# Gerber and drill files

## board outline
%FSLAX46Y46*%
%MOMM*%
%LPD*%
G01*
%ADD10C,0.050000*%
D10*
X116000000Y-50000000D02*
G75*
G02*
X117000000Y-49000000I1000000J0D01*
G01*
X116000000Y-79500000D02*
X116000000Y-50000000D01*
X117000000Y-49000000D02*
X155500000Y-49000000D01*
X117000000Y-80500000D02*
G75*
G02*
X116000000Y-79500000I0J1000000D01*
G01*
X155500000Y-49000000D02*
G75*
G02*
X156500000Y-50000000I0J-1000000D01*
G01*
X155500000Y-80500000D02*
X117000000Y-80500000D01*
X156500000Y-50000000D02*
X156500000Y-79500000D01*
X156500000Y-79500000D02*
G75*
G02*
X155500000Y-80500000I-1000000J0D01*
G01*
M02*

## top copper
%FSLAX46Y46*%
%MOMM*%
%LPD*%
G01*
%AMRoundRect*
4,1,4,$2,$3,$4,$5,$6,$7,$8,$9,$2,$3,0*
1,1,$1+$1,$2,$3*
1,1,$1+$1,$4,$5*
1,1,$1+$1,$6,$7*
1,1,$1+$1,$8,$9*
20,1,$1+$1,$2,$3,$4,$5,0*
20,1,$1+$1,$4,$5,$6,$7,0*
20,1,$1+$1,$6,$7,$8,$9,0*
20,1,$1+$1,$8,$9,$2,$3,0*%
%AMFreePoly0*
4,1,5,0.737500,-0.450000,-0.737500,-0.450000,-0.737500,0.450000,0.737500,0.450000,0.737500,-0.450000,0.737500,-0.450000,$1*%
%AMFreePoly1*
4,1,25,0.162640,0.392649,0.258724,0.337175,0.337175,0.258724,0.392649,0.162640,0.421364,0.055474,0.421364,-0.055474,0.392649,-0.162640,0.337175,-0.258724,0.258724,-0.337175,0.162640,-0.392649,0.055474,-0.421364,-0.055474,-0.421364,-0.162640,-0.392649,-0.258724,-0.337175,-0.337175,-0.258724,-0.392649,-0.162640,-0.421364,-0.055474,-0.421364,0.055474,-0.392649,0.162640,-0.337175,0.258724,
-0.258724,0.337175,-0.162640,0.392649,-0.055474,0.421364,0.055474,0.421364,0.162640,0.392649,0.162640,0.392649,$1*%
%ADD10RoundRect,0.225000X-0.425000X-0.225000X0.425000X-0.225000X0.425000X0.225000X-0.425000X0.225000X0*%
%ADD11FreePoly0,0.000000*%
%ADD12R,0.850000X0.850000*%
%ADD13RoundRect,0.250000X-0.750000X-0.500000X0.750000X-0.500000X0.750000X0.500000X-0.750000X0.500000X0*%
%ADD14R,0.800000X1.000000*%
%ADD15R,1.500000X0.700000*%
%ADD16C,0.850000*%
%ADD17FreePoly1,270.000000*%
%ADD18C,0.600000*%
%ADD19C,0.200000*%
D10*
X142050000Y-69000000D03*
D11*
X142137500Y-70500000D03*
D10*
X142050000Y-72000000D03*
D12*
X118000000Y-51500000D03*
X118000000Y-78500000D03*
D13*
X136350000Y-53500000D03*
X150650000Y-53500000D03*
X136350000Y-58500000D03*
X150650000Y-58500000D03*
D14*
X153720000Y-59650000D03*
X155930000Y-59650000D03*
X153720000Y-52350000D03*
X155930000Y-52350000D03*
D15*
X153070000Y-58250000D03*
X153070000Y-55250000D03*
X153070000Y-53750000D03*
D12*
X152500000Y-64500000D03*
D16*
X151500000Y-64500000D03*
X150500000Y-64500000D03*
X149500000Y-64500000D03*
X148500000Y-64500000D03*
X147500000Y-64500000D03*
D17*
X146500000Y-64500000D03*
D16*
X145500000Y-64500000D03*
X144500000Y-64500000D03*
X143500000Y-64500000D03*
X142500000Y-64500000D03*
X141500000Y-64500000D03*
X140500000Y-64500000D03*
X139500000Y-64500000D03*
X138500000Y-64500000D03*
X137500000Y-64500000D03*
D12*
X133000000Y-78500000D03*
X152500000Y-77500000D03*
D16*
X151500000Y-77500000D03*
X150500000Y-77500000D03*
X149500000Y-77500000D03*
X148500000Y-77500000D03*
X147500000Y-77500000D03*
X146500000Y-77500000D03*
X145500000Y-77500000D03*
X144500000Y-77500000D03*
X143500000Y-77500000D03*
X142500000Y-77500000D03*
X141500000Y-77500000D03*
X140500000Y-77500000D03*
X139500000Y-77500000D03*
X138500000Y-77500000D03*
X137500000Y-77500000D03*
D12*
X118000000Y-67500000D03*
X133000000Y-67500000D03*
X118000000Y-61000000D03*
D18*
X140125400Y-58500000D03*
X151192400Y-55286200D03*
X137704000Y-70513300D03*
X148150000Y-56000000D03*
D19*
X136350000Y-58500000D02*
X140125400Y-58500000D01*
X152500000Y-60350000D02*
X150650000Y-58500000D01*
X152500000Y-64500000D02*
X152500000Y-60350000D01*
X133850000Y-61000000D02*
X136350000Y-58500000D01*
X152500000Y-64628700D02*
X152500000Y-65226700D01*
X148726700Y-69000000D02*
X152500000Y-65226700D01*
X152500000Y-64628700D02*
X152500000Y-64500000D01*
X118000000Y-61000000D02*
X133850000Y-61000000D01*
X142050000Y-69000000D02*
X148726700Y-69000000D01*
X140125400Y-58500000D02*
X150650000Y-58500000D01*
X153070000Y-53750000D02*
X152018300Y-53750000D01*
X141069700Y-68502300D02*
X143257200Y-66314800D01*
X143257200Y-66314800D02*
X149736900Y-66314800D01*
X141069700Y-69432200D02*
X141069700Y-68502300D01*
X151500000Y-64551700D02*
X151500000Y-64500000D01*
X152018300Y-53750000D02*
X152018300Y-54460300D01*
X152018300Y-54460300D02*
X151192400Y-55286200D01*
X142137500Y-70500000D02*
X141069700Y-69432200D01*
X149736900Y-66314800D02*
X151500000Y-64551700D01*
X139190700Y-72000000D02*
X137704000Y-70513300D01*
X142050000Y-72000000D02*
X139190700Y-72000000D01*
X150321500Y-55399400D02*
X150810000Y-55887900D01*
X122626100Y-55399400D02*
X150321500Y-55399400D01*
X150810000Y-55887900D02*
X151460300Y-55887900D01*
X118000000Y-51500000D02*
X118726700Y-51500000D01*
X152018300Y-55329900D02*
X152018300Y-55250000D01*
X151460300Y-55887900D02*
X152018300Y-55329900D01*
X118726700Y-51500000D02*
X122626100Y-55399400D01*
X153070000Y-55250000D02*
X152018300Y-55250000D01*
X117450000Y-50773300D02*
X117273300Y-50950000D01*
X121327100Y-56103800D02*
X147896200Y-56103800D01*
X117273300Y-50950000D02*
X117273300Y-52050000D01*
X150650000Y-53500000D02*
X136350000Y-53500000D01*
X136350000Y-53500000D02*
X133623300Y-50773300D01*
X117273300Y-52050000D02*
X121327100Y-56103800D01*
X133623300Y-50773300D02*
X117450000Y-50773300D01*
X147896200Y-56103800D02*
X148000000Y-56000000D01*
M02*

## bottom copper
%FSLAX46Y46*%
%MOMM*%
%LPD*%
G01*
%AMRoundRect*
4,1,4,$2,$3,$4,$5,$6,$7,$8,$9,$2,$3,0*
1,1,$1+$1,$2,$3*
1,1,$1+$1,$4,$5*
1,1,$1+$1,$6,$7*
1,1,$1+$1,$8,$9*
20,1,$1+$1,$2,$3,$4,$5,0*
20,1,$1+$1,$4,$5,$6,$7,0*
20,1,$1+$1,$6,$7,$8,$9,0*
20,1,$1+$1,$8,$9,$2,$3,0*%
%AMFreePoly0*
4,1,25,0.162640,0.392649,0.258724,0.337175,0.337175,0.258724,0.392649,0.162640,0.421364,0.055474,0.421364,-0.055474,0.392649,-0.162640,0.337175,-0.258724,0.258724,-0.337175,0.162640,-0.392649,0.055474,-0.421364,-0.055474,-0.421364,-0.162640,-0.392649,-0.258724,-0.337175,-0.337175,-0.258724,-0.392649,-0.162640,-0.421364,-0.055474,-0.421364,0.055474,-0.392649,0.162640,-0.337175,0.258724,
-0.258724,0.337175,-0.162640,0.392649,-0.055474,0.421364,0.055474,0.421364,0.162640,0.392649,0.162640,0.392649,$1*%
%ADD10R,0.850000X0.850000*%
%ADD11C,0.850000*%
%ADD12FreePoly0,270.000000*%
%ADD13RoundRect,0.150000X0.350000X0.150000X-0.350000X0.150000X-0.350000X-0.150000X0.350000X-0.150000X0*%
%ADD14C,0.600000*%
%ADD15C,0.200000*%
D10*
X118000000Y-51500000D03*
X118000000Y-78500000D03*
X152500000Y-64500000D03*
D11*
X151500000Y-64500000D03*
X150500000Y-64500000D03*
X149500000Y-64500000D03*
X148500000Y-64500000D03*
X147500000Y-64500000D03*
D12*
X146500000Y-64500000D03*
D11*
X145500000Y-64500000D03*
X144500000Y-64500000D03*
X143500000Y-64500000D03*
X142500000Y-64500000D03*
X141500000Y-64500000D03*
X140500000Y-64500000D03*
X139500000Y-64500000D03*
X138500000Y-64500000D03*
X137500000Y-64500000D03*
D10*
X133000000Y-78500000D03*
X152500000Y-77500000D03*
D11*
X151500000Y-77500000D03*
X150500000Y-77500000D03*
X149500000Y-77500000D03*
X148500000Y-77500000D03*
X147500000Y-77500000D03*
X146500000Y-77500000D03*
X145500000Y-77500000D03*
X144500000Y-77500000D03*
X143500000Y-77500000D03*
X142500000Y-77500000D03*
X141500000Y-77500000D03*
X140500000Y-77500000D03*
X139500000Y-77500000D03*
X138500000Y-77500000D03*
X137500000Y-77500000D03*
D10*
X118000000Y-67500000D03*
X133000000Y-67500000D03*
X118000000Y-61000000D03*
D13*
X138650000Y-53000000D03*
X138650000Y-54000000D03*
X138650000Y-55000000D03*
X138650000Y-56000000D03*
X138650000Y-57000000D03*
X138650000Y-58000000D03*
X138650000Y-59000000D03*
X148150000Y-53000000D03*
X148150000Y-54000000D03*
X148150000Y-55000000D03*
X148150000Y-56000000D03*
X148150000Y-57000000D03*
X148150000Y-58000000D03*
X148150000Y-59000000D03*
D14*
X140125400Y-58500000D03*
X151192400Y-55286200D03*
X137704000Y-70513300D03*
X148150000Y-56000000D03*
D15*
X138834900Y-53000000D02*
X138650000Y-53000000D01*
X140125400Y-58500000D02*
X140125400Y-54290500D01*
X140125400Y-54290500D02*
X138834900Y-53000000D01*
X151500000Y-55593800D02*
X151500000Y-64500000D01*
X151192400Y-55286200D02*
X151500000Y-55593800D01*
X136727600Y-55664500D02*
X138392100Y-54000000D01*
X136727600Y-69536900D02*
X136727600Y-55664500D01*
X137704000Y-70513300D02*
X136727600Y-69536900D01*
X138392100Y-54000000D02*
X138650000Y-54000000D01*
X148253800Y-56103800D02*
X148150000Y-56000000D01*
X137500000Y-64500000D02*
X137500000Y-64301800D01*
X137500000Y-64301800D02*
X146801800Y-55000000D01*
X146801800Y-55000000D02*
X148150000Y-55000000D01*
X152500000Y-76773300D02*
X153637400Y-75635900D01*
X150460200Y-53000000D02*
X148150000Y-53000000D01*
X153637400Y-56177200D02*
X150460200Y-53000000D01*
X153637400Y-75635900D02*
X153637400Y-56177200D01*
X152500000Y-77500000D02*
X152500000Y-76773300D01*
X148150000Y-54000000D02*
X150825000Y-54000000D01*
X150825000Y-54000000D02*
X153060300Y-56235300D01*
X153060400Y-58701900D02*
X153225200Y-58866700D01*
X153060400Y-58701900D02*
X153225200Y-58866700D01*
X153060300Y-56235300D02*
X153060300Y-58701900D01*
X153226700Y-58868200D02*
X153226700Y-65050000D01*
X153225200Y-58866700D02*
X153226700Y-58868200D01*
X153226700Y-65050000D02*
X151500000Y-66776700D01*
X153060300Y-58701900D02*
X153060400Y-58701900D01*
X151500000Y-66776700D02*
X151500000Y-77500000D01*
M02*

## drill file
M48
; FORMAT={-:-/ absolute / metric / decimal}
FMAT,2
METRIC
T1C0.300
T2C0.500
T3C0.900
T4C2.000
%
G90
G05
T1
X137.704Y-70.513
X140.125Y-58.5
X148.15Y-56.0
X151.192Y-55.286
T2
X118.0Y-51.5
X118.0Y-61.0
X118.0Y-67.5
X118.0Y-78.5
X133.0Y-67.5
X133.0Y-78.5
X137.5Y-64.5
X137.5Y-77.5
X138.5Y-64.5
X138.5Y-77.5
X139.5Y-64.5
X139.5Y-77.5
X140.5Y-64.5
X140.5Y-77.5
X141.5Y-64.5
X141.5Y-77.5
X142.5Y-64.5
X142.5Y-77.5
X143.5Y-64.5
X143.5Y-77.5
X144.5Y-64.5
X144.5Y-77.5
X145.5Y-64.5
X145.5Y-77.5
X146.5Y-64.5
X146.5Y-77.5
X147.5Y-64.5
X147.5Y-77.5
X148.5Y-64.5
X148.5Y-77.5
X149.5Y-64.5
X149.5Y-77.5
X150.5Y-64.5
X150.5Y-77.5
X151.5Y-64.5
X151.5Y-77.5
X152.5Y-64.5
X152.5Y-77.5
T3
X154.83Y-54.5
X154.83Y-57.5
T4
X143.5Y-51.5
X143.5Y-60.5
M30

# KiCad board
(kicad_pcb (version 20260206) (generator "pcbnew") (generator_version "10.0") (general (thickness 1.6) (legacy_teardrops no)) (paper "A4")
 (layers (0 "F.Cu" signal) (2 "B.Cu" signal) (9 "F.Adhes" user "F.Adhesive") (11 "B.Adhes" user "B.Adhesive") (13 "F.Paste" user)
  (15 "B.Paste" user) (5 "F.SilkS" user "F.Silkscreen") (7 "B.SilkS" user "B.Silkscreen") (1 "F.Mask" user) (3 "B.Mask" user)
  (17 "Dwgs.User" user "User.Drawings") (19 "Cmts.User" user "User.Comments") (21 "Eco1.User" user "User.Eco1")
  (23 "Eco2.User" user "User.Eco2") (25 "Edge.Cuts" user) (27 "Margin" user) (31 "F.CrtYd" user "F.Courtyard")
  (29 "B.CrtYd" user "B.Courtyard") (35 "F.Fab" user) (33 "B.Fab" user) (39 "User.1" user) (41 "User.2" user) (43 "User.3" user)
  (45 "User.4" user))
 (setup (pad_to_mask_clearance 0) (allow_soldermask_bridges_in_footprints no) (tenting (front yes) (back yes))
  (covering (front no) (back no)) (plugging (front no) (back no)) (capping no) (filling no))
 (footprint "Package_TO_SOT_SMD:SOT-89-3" (layer "F.Cu") (at 144 70.5)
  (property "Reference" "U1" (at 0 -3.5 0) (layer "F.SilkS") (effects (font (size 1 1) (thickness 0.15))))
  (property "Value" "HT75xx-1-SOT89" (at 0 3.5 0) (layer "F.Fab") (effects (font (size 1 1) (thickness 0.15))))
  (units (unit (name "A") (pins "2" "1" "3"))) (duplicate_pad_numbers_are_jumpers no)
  (pad "1" smd roundrect (at -1.95 -1.5) (size 1.3 0.9) (layers "F.Cu" "F.Mask" "F.Paste") (roundrect_rratio 0.25) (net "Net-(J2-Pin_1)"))
  (pad "2" smd custom (at -1.8625 0) (size 1.475 0.9) (layers "F.Cu" "F.Mask" "F.Paste") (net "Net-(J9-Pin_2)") (zone_connect 2)
   (thermal_bridge_angle 45) (options (clearance outline) (anchor rect)) (primitives))
  (pad "3" smd roundrect (at -1.95 1.5) (size 1.3 0.9) (layers "F.Cu" "F.Mask" "F.Paste") (roundrect_rratio 0.25) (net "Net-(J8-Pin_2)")))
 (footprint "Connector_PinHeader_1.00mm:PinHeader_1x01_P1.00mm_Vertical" (layer "F.Cu") (at 118 51.5 90)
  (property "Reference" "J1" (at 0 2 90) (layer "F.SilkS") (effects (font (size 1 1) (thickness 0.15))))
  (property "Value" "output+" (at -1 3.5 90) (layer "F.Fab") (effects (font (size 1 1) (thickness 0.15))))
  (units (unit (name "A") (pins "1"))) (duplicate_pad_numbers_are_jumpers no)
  (pad "1" thru_hole rect (at 0 0 90) (size 0.85 0.85) (drill 0.5) (layers "*.Cu" "*.Mask") (remove_unused_layers no) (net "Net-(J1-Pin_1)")))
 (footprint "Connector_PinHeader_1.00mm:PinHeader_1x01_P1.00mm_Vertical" (layer "F.Cu") (at 118 78.5 90)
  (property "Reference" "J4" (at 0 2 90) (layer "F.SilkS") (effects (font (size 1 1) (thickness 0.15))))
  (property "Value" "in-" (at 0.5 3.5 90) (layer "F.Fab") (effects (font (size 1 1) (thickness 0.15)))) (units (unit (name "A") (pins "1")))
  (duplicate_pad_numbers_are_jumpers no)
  (pad "1" thru_hole rect (at 0 0 90) (size 0.85 0.85) (drill 0.5) (layers "*.Cu" "*.Mask") (remove_unused_layers no)
   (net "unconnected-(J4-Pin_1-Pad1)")))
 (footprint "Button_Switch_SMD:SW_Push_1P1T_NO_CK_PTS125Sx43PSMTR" (layer "F.Cu") (at 143.5 56)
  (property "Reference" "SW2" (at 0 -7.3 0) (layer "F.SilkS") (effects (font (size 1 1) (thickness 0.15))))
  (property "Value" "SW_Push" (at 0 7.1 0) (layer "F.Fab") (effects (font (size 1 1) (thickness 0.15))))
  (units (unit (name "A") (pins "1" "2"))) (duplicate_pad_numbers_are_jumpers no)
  (pad "" np_thru_hole circle (at 0 -4.5) (size 2 2) (drill 2) (layers "*.Cu" "*.Mask"))
  (pad "" np_thru_hole circle (at 0 4.5) (size 2 2) (drill 2) (layers "*.Cu" "*.Mask"))
  (pad "1" smd roundrect (at -7.15 -2.5) (size 2 1.5) (layers "F.Cu" "F.Mask" "F.Paste") (roundrect_rratio 0.1666666667)
   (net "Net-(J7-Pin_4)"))
  (pad "1" smd roundrect (at 7.15 -2.5) (size 2 1.5) (layers "F.Cu" "F.Mask" "F.Paste") (roundrect_rratio 0.1666666667)
   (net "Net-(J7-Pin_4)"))
  (pad "2" smd roundrect (at -7.15 2.5) (size 2 1.5) (layers "F.Cu" "F.Mask" "F.Paste") (roundrect_rratio 0.1666666667)
   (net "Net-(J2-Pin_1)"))
  (pad "2" smd roundrect (at 7.15 2.5) (size 2 1.5) (layers "F.Cu" "F.Mask" "F.Paste") (roundrect_rratio 0.1666666667)
   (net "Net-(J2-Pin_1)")))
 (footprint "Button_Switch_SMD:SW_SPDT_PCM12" (layer "F.Cu") (at 154.5 56 90)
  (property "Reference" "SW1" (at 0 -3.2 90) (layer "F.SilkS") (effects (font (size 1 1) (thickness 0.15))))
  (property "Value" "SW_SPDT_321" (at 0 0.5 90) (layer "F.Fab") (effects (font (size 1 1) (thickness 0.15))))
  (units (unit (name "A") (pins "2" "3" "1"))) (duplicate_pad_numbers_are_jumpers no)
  (pad "" smd rect (at -3.65 -0.78 90) (size 1 0.8) (layers "F.Cu" "F.Mask" "F.Paste"))
  (pad "" smd rect (at -3.65 1.43 90) (size 1 0.8) (layers "F.Cu" "F.Mask" "F.Paste"))
  (pad "" np_thru_hole circle (at -1.5 0.33 90) (size 0.9 0.9) (drill 0.9) (layers "*.Cu" "*.Mask"))
  (pad "" np_thru_hole circle (at 1.5 0.33 90) (size 0.9 0.9) (drill 0.9) (layers "*.Cu" "*.Mask"))
  (pad "" smd rect (at 3.65 -0.78 90) (size 1 0.8) (layers "F.Cu" "F.Mask" "F.Paste"))
  (pad "" smd rect (at 3.65 1.43 90) (size 1 0.8) (layers "F.Cu" "F.Mask" "F.Paste"))
  (pad "1" smd rect (at -2.25 -1.43 90) (size 0.7 1.5) (layers "F.Cu" "F.Mask" "F.Paste") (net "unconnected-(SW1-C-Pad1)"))
  (pad "2" smd rect (at 0.75 -1.43 90) (size 0.7 1.5) (layers "F.Cu" "F.Mask" "F.Paste") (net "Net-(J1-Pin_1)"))
  (pad "3" smd rect (at 2.25 -1.43 90) (size 0.7 1.5) (layers "F.Cu" "F.Mask" "F.Paste") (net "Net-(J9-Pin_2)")))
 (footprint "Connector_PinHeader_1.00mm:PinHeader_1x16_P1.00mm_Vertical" (layer "F.Cu") (at 152.5 64.5 -90)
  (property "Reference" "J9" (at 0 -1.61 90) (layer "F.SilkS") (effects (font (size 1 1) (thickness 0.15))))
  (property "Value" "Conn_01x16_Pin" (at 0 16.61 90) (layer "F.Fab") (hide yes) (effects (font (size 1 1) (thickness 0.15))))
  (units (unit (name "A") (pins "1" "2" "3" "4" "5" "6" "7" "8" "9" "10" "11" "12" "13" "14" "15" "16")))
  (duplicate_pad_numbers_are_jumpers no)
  (pad "1" thru_hole rect (at 0 0 270) (size 0.85 0.85) (drill 0.5) (layers "*.Cu" "*.Mask") (remove_unused_layers no)
   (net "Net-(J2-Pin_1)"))
  (pad "2" thru_hole circle (at 0 1 270) (size 0.85 0.85) (drill 0.5) (layers "*.Cu" "*.Mask") (remove_unused_layers no)
   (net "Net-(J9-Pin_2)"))
  (pad "3" thru_hole circle (at 0 2 270) (size 0.85 0.85) (drill 0.5) (layers "*.Cu" "*.Mask") (remove_unused_layers no)
   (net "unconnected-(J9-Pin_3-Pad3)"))
  (pad "4" thru_hole circle (at 0 3 270) (size 0.85 0.85) (drill 0.5) (layers "*.Cu" "*.Mask") (remove_unused_layers no)
   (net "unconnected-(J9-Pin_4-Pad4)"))
  (pad "5" thru_hole circle (at 0 4 270) (size 0.85 0.85) (drill 0.5) (layers "*.Cu" "*.Mask") (remove_unused_layers no)
   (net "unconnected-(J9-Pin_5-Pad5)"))
  (pad "6" thru_hole circle (at 0 5 270) (size 0.85 0.85) (drill 0.5) (layers "*.Cu" "*.Mask") (remove_unused_layers no)
   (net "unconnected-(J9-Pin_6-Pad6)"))
  (pad "7" thru_hole custom (at 0 6 270) (size 0.85 0.85) (drill 0.5) (layers "*.Cu" "*.Mask") (remove_unused_layers no)
   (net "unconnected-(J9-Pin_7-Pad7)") (thermal_bridge_angle 90) (options (clearance outline) (anchor circle)) (primitives))
  (pad "8" thru_hole circle (at 0 7 270) (size 0.85 0.85) (drill 0.5) (layers "*.Cu" "*.Mask") (remove_unused_layers no)
   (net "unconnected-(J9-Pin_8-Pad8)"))
  (pad "9" thru_hole circle (at 0 8 270) (size 0.85 0.85) (drill 0.5) (layers "*.Cu" "*.Mask") (remove_unused_layers no)
   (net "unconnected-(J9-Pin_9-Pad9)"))
  (pad "10" thru_hole circle (at 0 9 270) (size 0.85 0.85) (drill 0.5) (layers "*.Cu" "*.Mask") (remove_unused_layers no)
   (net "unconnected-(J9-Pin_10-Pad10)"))
  (pad "11" thru_hole circle (at 0 10 270) (size 0.85 0.85) (drill 0.5) (layers "*.Cu" "*.Mask") (remove_unused_layers no)
   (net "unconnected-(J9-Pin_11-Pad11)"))
  (pad "12" thru_hole circle (at 0 11 270) (size 0.85 0.85) (drill 0.5) (layers "*.Cu" "*.Mask") (remove_unused_layers no)
   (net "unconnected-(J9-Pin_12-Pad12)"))
  (pad "13" thru_hole circle (at 0 12 270) (size 0.85 0.85) (drill 0.5) (layers "*.Cu" "*.Mask") (remove_unused_layers no)
   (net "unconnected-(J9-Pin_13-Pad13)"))
  (pad "14" thru_hole circle (at 0 13 270) (size 0.85 0.85) (drill 0.5) (layers "*.Cu" "*.Mask") (remove_unused_layers no)
   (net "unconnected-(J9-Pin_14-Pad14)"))
  (pad "15" thru_hole circle (at 0 14 270) (size 0.85 0.85) (drill 0.5) (layers "*.Cu" "*.Mask") (remove_unused_layers no)
   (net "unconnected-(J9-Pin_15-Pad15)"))
  (pad "16" thru_hole circle (at 0 15 270) (size 0.85 0.85) (drill 0.5) (layers "*.Cu" "*.Mask") (remove_unused_layers no)
   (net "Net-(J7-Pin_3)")))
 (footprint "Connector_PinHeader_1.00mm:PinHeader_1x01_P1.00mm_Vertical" (layer "F.Cu") (at 133 78.5 90)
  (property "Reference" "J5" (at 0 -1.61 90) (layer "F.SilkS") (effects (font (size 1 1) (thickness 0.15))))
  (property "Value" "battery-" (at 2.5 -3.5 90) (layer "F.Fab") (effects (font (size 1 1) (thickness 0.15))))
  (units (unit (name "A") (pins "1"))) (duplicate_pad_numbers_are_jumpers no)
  (pad "1" thru_hole rect (at 0 0 90) (size 0.85 0.85) (drill 0.5) (layers "*.Cu" "*.Mask") (remove_unused_layers no)
   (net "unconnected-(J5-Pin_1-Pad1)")))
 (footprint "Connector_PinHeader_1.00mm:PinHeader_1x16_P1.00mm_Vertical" (layer "F.Cu") (at 152.5 77.5 -90)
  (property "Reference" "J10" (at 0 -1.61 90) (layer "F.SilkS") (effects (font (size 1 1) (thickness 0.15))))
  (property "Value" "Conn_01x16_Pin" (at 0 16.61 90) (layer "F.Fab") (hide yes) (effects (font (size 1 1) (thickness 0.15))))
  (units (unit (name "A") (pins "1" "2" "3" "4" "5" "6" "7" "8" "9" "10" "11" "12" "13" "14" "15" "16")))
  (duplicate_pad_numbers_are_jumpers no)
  (pad "1" thru_hole rect (at 0 0 270) (size 0.85 0.85) (drill 0.5) (layers "*.Cu" "*.Mask") (remove_unused_layers no)
   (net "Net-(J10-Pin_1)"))
  (pad "2" thru_hole circle (at 0 1 270) (size 0.85 0.85) (drill 0.5) (layers "*.Cu" "*.Mask") (remove_unused_layers no)
   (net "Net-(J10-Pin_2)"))
  (pad "3" thru_hole circle (at 0 2 270) (size 0.85 0.85) (drill 0.5) (layers "*.Cu" "*.Mask") (remove_unused_layers no)
   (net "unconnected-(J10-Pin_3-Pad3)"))
  (pad "4" thru_hole circle (at 0 3 270) (size 0.85 0.85) (drill 0.5) (layers "*.Cu" "*.Mask") (remove_unused_layers no)
   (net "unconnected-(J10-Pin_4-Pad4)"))
  (pad "5" thru_hole circle (at 0 4 270) (size 0.85 0.85) (drill 0.5) (layers "*.Cu" "*.Mask") (remove_unused_layers no)
   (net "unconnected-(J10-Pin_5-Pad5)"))
  (pad "6" thru_hole circle (at 0 5 270) (size 0.85 0.85) (drill 0.5) (layers "*.Cu" "*.Mask") (remove_unused_layers no)
   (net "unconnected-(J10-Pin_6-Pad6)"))
  (pad "7" thru_hole circle (at 0 6 270) (size 0.85 0.85) (drill 0.5) (layers "*.Cu" "*.Mask") (remove_unused_layers no)
   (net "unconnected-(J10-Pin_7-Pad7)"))
  (pad "8" thru_hole circle (at 0 7 270) (size 0.85 0.85) (drill 0.5) (layers "*.Cu" "*.Mask") (remove_unused_layers no)
   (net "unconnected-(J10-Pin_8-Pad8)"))
  (pad "9" thru_hole circle (at 0 8 270) (size 0.85 0.85) (drill 0.5) (layers "*.Cu" "*.Mask") (remove_unused_layers no)
   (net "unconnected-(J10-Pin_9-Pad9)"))
  (pad "10" thru_hole circle (at 0 9 270) (size 0.85 0.85) (drill 0.5) (layers "*.Cu" "*.Mask") (remove_unused_layers no)
   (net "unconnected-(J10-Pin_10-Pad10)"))
  (pad "11" thru_hole circle (at 0 10 270) (size 0.85 0.85) (drill 0.5) (layers "*.Cu" "*.Mask") (remove_unused_layers no)
   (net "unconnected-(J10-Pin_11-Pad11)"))
  (pad "12" thru_hole circle (at 0 11 270) (size 0.85 0.85) (drill 0.5) (layers "*.Cu" "*.Mask") (remove_unused_layers no)
   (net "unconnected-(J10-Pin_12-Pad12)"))
  (pad "13" thru_hole circle (at 0 12 270) (size 0.85 0.85) (drill 0.5) (layers "*.Cu" "*.Mask") (remove_unused_layers no)
   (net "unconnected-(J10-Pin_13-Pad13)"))
  (pad "14" thru_hole circle (at 0 13 270) (size 0.85 0.85) (drill 0.5) (layers "*.Cu" "*.Mask") (remove_unused_layers no)
   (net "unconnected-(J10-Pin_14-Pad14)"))
  (pad "15" thru_hole circle (at 0 14 270) (size 0.85 0.85) (drill 0.5) (layers "*.Cu" "*.Mask") (remove_unused_layers no)
   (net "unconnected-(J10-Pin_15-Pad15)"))
  (pad "16" thru_hole circle (at 0 15 270) (size 0.85 0.85) (drill 0.5) (layers "*.Cu" "*.Mask") (remove_unused_layers no)
   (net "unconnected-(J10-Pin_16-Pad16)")))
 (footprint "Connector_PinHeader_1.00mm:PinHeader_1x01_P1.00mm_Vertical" (layer "F.Cu") (at 118 67.5 90)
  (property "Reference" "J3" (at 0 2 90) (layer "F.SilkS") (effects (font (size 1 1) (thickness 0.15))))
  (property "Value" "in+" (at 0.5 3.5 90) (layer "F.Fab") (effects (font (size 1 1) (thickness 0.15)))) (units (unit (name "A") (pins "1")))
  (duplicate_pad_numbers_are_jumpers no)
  (pad "1" thru_hole rect (at 0 0 90) (size 0.85 0.85) (drill 0.5) (layers "*.Cu" "*.Mask") (remove_unused_layers no)
   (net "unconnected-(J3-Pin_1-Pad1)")))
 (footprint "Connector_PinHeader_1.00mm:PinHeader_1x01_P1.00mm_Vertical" (layer "F.Cu") (at 133 67.5 90)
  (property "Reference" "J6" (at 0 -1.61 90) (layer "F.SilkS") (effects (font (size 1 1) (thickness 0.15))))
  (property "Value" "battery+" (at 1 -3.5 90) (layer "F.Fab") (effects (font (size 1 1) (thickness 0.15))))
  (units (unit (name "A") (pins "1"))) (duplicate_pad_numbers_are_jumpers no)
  (pad "1" thru_hole rect (at 0 0 90) (size 0.85 0.85) (drill 0.5) (layers "*.Cu" "*.Mask") (remove_unused_layers no)
   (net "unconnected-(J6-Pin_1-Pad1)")))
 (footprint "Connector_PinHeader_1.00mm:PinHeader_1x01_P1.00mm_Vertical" (layer "F.Cu") (at 118 61 90)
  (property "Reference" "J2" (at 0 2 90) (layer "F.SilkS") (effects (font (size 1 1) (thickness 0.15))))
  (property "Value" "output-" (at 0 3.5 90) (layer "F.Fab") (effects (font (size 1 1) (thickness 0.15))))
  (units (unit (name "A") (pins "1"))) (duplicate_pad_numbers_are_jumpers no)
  (pad "1" thru_hole rect (at 0 0 90) (size 0.85 0.85) (drill 0.5) (layers "*.Cu" "*.Mask") (remove_unused_layers no) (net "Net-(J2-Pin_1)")))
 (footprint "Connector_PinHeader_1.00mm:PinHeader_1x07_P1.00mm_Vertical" (layer "B.Cu") (at 138.65 53 180)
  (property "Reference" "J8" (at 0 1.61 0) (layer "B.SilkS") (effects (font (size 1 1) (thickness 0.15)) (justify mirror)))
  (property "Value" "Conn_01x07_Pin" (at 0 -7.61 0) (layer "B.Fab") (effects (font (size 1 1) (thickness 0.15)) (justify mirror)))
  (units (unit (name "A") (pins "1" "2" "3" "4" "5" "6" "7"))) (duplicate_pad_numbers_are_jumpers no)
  (pad "1" smd roundrect (at 0 0 180) (size 1 0.6) (layers "B.Cu" "B.Mask" "B.Paste") (roundrect_rratio 0.25) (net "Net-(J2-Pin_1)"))
  (pad "2" smd roundrect (at 0 -1 180) (size 1 0.6) (layers "B.Cu" "B.Mask" "B.Paste") (roundrect_rratio 0.25) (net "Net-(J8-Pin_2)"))
  (pad "3" smd roundrect (at 0 -2 180) (size 1 0.6) (layers "B.Cu" "B.Mask" "B.Paste") (roundrect_rratio 0.25)
   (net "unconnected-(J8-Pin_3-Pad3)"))
  (pad "4" smd roundrect (at 0 -3 180) (size 1 0.6) (layers "B.Cu" "B.Mask" "B.Paste") (roundrect_rratio 0.25)
   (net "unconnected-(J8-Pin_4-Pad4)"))
  (pad "5" smd roundrect (at 0 -4 180) (size 1 0.6) (layers "B.Cu" "B.Mask" "B.Paste") (roundrect_rratio 0.25)
   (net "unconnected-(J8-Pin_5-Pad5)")
   (teardrops (best_length_ratio 0.5) (max_length 1) (best_width_ratio 1) (max_width 2) (curved_edges no) (filter_ratio 1) (enabled no)
    (allow_two_segments yes) (prefer_zone_connections yes)))
  (pad "6" smd roundrect (at 0 -5 180) (size 1 0.6) (layers "B.Cu" "B.Mask" "B.Paste") (roundrect_rratio 0.25)
   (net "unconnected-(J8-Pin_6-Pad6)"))
  (pad "7" smd roundrect (at 0 -6 180) (size 1 0.6) (layers "B.Cu" "B.Mask" "B.Paste") (roundrect_rratio 0.25)
   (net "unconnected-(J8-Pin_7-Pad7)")))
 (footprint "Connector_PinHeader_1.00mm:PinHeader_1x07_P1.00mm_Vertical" (layer "B.Cu") (at 148.15 53 180)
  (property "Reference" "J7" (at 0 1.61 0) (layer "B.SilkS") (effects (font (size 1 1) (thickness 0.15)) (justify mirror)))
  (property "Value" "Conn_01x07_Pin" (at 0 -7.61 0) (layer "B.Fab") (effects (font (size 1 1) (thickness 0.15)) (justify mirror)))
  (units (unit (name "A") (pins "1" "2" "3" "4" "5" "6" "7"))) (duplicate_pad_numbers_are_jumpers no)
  (pad "1" smd roundrect (at 0 0 180) (size 1 0.6) (layers "B.Cu" "B.Mask" "B.Paste") (roundrect_rratio 0.25) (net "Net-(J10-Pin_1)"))
  (pad "2" smd roundrect (at 0 -1 180) (size 1 0.6) (layers "B.Cu" "B.Mask" "B.Paste") (roundrect_rratio 0.25) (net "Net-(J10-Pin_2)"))
  (pad "3" smd roundrect (at 0 -2 180) (size 1 0.6) (layers "B.Cu" "B.Mask" "B.Paste") (roundrect_rratio 0.25) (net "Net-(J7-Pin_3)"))
  (pad "4" smd roundrect (at 0 -3 180) (size 1 0.6) (layers "B.Cu" "B.Mask" "B.Paste") (roundrect_rratio 0.25) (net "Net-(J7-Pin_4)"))
  (pad "5" smd roundrect (at 0 -4 180) (size 1 0.6) (layers "B.Cu" "B.Mask" "B.Paste") (roundrect_rratio 0.25)
   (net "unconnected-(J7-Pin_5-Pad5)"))
  (pad "6" smd roundrect (at 0 -5 180) (size 1 0.6) (layers "B.Cu" "B.Mask" "B.Paste") (roundrect_rratio 0.25)
   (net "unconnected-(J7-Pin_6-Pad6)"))
  (pad "7" smd roundrect (at 0 -6 180) (size 1 0.6) (layers "B.Cu" "B.Mask" "B.Paste") (roundrect_rratio 0.25)
   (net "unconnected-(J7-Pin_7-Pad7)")))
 (gr_arc (start 116 50) (mid 116.292893 49.292893) (end 117 49) (stroke (width 0.05) (type default)) (layer "Edge.Cuts"))
 (gr_line (start 116 79.5) (end 116 50) (stroke (width 0.05) (type default)) (layer "Edge.Cuts"))
 (gr_line (start 117 49) (end 155.5 49) (stroke (width 0.05) (type default)) (layer "Edge.Cuts"))
 (gr_arc (start 117 80.5) (mid 116.292893 80.207107) (end 116 79.5) (stroke (width 0.05) (type default)) (layer "Edge.Cuts"))
 (gr_arc (start 155.5 49) (mid 156.207107 49.292893) (end 156.5 50) (stroke (width 0.05) (type default)) (layer "Edge.Cuts"))
 (gr_line (start 155.5 80.5) (end 117 80.5) (stroke (width 0.05) (type default)) (layer "Edge.Cuts"))
 (gr_line (start 156.5 50) (end 156.5 79.5) (stroke (width 0.05) (type default)) (layer "Edge.Cuts"))
 (gr_arc (start 156.5 79.5) (mid 156.207107 80.207107) (end 155.5 80.5) (stroke (width 0.05) (type default)) (layer "Edge.Cuts"))
 (segment (start 136.35 58.5) (end 140.1254 58.5) (width 0.2) (layer "F.Cu") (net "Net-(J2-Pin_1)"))
 (segment (start 152.5 60.35) (end 150.65 58.5) (width 0.2) (layer "F.Cu") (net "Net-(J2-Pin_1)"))
 (segment (start 152.5 64.5) (end 152.5 60.35) (width 0.2) (layer "F.Cu") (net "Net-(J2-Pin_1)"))
 (segment (start 133.85 61) (end 136.35 58.5) (width 0.2) (layer "F.Cu") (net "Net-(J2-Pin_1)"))
 (segment (start 152.5 64.6287) (end 152.5 65.2267) (width 0.2) (layer "F.Cu") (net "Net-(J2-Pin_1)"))
 (segment (start 148.7267 69) (end 152.5 65.2267) (width 0.2) (layer "F.Cu") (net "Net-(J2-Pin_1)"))
 (segment (start 152.5 64.6287) (end 152.5 64.5) (width 0.2) (layer "F.Cu") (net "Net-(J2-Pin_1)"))
 (segment (start 118 61) (end 133.85 61) (width 0.2) (layer "F.Cu") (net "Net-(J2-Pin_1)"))
 (segment (start 142.05 69) (end 148.7267 69) (width 0.2) (layer "F.Cu") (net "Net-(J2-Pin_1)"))
 (segment (start 140.1254 58.5) (end 150.65 58.5) (width 0.2) (layer "F.Cu") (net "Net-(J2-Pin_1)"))
 (via (at 140.1254 58.5) (size 0.6) (drill 0.3) (layers "F.Cu" "B.Cu") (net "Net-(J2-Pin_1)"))
 (segment (start 138.8349 53) (end 138.65 53) (width 0.2) (layer "B.Cu") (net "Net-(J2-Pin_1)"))
 (segment (start 140.1254 58.5) (end 140.1254 54.2905) (width 0.2) (layer "B.Cu") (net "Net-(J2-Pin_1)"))
 (segment (start 140.1254 54.2905) (end 138.8349 53) (width 0.2) (layer "B.Cu") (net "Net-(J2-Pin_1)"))
 (segment (start 153.07 53.75) (end 152.0183 53.75) (width 0.2) (layer "F.Cu") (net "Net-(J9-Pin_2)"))
 (segment (start 141.0697 68.5023) (end 143.2572 66.3148) (width 0.2) (layer "F.Cu") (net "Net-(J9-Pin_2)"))
 (segment (start 143.2572 66.3148) (end 149.7369 66.3148) (width 0.2) (layer "F.Cu") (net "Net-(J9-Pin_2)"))
 (segment (start 141.0697 69.4322) (end 141.0697 68.5023) (width 0.2) (layer "F.Cu") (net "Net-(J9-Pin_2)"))
 (segment (start 151.5 64.5517) (end 151.5 64.5) (width 0.2) (layer "F.Cu") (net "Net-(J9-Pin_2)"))
 (segment (start 152.0183 53.75) (end 152.0183 54.4603) (width 0.2) (layer "F.Cu") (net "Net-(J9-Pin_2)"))
 (segment (start 152.0183 54.4603) (end 151.1924 55.2862) (width 0.2) (layer "F.Cu") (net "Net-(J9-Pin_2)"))
 (segment (start 142.1375 70.5) (end 141.0697 69.4322) (width 0.2) (layer "F.Cu") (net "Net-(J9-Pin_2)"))
 (segment (start 149.7369 66.3148) (end 151.5 64.5517) (width 0.2) (layer "F.Cu") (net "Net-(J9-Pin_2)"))
 (via (at 151.1924 55.2862) (size 0.6) (drill 0.3) (layers "F.Cu" "B.Cu") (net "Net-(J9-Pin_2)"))
 (segment (start 151.5 55.5938) (end 151.5 64.5) (width 0.2) (layer "B.Cu") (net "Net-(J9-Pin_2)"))
 (segment (start 151.1924 55.2862) (end 151.5 55.5938) (width 0.2) (layer "B.Cu") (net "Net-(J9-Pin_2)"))
 (segment (start 139.1907 72) (end 137.704 70.5133) (width 0.2) (layer "F.Cu") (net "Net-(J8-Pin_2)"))
 (segment (start 142.05 72) (end 139.1907 72) (width 0.2) (layer "F.Cu") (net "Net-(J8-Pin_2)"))
 (via (at 137.704 70.5133) (size 0.6) (drill 0.3) (layers "F.Cu" "B.Cu") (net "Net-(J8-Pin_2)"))
 (segment (start 136.7276 55.6645) (end 138.3921 54) (width 0.2) (layer "B.Cu") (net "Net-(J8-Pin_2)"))
 (segment (start 136.7276 69.5369) (end 136.7276 55.6645) (width 0.2) (layer "B.Cu") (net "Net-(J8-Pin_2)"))
 (segment (start 137.704 70.5133) (end 136.7276 69.5369) (width 0.2) (layer "B.Cu") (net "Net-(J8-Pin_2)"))
 (segment (start 138.3921 54) (end 138.65 54) (width 0.2) (layer "B.Cu") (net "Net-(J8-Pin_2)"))
 (segment (start 150.3215 55.3994) (end 150.81 55.8879) (width 0.2) (layer "F.Cu") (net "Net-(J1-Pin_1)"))
 (segment (start 122.6261 55.3994) (end 150.3215 55.3994) (width 0.2) (layer "F.Cu") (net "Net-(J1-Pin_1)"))
 (segment (start 150.81 55.8879) (end 151.4603 55.8879) (width 0.2) (layer "F.Cu") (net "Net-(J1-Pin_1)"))
 (segment (start 118 51.5) (end 118.7267 51.5) (width 0.2) (layer "F.Cu") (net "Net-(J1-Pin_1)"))
 (segment (start 152.0183 55.3299) (end 152.0183 55.25) (width 0.2) (layer "F.Cu") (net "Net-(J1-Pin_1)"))
 (segment (start 151.4603 55.8879) (end 152.0183 55.3299) (width 0.2) (layer "F.Cu") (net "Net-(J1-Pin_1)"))
 (segment (start 118.7267 51.5) (end 122.6261 55.3994) (width 0.2) (layer "F.Cu") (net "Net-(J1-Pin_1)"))
 (segment (start 153.07 55.25) (end 152.0183 55.25) (width 0.2) (layer "F.Cu") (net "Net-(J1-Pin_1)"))
 (segment (start 117.45 50.7733) (end 117.2733 50.95) (width 0.2) (layer "F.Cu") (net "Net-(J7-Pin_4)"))
 (segment (start 121.3271 56.1038) (end 147.8962 56.1038) (width 0.2) (layer "F.Cu") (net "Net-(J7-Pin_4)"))
 (segment (start 117.2733 50.95) (end 117.2733 52.05) (width 0.2) (layer "F.Cu") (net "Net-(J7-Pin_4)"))
 (segment (start 150.65 53.5) (end 136.35 53.5) (width 0.2) (layer "F.Cu") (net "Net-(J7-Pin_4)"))
 (segment (start 136.35 53.5) (end 133.6233 50.7733) (width 0.2) (layer "F.Cu") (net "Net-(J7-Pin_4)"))
 (segment (start 117.2733 52.05) (end 121.3271 56.1038) (width 0.2) (layer "F.Cu") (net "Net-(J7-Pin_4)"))
 (segment (start 133.6233 50.7733) (end 117.45 50.7733) (width 0.2) (layer "F.Cu") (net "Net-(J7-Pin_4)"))
 (segment (start 147.8962 56.1038) (end 148 56) (width 0.2) (layer "F.Cu") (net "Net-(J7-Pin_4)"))
 (via (at 148.15 56) (size 0.6) (drill 0.3) (layers "F.Cu" "B.Cu") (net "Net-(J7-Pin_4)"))
 (segment (start 148.2538 56.1038) (end 148.15 56) (width 0.2) (layer "B.Cu") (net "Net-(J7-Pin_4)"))
 (segment (start 137.5 64.5) (end 137.5 64.3018) (width 0.2) (layer "B.Cu") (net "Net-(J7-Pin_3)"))
 (segment (start 137.5 64.3018) (end 146.8018 55) (width 0.2) (layer "B.Cu") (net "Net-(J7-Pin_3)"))
 (segment (start 146.8018 55) (end 148.15 55) (width 0.2) (layer "B.Cu") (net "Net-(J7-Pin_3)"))
 (segment (start 152.5 76.7733) (end 153.6374 75.6359) (width 0.2) (layer "B.Cu") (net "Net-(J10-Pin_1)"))
 (segment (start 150.4602 53) (end 148.15 53) (width 0.2) (layer "B.Cu") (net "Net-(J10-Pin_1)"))
 (segment (start 153.6374 56.1772) (end 150.4602 53) (width 0.2) (layer "B.Cu") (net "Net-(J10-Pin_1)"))
 (segment (start 153.6374 75.6359) (end 153.6374 56.1772) (width 0.2) (layer "B.Cu") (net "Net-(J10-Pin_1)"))
 (segment (start 152.5 77.5) (end 152.5 76.7733) (width 0.2) (layer "B.Cu") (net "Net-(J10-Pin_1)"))
 (segment (start 148.15 54) (end 150.825 54) (width 0.2) (layer "B.Cu") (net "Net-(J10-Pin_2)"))
 (segment (start 150.825 54) (end 153.0603 56.2353) (width 0.2) (layer "B.Cu") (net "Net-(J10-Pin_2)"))
 (segment (start 153.0604 58.7019) (end 153.2252 58.8667) (width 0.2) (layer "B.Cu") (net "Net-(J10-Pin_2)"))
 (segment (start 153.0604 58.7019) (end 153.2252 58.8667) (width 0.2) (layer "B.Cu") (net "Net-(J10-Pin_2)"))
 (segment (start 153.0603 56.2353) (end 153.0603 58.7019) (width 0.2) (layer "B.Cu") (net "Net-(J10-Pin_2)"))
 (segment (start 153.2267 58.8682) (end 153.2267 65.05) (width 0.2) (layer "B.Cu") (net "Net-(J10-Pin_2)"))
 (segment (start 153.2252 58.8667) (end 153.2267 58.8682) (width 0.2) (layer "B.Cu") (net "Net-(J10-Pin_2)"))
 (segment (start 153.2267 65.05) (end 151.5 66.7767) (width 0.2) (layer "B.Cu") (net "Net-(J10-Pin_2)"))
 (segment (start 153.0603 58.7019) (end 153.0604 58.7019) (width 0.2) (layer "B.Cu") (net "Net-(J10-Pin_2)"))
 (segment (start 151.5 66.7767) (end 151.5 77.5) (width 0.2) (layer "B.Cu") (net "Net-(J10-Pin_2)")))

